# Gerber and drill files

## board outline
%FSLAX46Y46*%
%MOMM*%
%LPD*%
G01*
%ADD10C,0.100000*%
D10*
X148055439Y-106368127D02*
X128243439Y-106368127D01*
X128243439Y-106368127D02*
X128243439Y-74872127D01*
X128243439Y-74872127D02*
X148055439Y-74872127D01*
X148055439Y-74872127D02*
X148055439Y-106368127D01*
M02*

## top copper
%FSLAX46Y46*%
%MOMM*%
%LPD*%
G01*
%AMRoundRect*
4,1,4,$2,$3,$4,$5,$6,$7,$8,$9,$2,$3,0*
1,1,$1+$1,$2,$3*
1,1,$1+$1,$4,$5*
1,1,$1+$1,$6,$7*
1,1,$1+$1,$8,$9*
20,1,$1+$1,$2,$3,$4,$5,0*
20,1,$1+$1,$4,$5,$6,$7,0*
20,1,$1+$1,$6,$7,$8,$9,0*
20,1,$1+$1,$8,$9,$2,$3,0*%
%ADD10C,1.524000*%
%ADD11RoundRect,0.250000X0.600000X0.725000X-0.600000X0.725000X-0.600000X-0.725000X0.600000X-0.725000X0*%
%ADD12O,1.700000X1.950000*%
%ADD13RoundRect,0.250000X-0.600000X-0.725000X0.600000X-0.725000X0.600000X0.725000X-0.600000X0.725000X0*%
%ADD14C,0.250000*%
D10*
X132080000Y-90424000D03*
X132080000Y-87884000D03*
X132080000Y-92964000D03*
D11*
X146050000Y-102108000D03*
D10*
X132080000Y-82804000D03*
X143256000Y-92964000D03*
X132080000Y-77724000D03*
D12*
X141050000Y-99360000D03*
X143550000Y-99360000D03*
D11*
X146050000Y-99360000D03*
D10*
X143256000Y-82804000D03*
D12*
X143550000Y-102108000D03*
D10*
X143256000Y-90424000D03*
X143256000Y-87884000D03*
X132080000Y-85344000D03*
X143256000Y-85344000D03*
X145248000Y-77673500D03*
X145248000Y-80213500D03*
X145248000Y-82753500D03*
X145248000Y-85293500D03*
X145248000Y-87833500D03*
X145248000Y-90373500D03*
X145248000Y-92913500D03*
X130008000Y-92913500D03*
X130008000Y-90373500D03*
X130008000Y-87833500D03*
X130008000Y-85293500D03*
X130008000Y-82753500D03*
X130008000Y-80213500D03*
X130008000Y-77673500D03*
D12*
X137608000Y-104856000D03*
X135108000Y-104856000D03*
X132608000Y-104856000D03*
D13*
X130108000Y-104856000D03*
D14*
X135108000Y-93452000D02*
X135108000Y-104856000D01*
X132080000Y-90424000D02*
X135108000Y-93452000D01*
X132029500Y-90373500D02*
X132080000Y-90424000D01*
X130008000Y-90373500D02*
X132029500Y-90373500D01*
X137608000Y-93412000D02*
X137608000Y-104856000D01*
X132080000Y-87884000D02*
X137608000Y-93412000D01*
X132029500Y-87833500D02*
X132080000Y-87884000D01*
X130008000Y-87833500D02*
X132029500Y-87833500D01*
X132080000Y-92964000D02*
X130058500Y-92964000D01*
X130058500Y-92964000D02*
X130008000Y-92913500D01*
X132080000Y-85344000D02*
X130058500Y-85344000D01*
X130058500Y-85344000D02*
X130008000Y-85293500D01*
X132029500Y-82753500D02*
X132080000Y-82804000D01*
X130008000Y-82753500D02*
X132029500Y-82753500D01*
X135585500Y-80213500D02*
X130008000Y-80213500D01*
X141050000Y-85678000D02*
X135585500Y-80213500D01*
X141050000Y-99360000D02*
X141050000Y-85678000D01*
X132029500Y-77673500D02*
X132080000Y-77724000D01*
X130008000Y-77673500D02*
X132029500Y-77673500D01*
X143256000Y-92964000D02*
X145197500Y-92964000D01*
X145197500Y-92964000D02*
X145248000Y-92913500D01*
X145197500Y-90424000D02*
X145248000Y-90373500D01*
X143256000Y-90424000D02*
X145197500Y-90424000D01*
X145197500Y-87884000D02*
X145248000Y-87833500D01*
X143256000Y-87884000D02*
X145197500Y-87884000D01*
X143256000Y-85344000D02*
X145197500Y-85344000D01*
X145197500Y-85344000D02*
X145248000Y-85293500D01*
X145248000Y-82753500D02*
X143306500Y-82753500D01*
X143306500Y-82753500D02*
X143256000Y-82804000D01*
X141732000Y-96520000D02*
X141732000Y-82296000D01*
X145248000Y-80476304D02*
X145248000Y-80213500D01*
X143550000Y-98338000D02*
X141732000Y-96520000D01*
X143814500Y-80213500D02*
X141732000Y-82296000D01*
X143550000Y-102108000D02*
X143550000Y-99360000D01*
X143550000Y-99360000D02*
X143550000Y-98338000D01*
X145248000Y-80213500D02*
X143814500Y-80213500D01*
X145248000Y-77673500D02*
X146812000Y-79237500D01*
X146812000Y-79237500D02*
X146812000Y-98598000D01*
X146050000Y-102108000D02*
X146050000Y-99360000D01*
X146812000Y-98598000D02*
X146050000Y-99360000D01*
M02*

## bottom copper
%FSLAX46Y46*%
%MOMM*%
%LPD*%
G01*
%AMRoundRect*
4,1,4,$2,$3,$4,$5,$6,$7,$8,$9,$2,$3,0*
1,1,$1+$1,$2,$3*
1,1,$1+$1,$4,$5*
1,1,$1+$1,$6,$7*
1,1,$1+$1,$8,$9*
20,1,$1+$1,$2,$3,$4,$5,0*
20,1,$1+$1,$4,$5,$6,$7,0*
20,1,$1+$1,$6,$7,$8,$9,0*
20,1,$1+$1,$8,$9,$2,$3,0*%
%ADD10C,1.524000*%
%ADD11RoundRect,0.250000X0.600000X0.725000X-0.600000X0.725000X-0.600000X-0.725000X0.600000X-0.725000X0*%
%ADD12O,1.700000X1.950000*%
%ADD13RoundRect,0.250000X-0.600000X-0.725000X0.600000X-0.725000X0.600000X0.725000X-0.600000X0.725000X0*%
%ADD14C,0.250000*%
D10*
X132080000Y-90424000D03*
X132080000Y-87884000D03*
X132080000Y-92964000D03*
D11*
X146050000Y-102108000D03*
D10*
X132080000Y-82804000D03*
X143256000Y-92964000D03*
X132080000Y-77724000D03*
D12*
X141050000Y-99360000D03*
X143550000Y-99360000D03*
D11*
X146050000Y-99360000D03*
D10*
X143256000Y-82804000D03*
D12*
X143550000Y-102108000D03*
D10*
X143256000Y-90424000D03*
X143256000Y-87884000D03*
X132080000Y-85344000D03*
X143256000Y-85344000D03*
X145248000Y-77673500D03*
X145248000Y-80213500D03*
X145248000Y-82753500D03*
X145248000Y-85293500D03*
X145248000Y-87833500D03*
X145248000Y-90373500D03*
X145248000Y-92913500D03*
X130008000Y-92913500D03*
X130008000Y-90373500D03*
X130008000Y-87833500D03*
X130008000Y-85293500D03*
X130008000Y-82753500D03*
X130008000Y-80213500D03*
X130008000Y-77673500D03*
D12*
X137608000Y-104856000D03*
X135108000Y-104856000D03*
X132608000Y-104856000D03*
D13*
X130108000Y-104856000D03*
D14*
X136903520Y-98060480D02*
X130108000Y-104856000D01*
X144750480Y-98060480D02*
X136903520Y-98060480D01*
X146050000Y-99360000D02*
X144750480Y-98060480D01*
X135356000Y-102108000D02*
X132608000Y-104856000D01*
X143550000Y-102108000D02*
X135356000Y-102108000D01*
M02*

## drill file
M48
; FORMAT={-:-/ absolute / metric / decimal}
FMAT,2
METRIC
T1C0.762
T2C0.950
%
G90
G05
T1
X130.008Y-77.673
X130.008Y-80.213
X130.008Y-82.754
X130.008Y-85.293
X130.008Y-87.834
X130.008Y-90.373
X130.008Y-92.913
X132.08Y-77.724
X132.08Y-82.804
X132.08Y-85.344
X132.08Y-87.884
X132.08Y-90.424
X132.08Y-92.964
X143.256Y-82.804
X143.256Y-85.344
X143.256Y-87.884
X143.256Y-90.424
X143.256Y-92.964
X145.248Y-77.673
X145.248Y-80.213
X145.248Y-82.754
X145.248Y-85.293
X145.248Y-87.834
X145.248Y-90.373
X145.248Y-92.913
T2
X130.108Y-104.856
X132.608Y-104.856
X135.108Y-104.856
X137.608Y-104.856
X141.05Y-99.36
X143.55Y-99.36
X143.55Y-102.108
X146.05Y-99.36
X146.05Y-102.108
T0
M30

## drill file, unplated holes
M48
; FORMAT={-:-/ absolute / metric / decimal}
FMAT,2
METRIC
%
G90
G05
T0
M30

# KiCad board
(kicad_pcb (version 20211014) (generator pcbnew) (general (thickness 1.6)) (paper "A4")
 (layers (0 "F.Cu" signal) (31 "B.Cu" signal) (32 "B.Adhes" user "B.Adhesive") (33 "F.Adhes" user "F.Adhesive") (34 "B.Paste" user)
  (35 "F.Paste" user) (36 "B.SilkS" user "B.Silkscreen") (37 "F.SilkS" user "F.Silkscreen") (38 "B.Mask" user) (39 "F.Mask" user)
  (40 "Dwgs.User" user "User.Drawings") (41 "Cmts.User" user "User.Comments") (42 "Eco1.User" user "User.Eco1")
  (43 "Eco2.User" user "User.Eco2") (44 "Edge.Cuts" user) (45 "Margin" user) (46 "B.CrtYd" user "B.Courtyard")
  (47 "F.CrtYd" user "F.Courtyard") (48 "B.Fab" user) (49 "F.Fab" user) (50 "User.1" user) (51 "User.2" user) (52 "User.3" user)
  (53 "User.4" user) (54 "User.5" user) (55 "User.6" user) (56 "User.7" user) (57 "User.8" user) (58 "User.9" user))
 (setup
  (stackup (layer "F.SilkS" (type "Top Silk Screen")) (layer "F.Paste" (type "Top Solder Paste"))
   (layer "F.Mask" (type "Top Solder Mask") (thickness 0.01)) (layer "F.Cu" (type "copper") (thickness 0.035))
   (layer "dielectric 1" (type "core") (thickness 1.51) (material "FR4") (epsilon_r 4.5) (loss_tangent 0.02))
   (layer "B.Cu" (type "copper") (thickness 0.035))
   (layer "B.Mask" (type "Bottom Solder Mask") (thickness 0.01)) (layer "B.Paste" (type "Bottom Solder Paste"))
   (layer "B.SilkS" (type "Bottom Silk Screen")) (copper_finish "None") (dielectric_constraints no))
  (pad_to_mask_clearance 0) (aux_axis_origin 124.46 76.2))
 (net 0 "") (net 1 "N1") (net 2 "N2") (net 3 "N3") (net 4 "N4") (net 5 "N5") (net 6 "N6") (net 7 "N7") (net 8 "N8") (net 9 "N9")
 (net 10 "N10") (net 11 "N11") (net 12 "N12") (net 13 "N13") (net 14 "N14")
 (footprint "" (layer "F.Cu") (at 132.08 92.964)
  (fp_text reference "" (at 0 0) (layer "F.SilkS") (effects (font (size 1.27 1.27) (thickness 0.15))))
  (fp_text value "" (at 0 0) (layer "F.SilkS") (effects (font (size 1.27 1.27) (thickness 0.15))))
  (pad "7" thru_hole circle (at 0 0) (size 1.524 1.524) (drill 0.762) (layers *.Cu *.Mask) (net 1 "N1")))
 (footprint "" (layer "F.Cu") (at 146.05 102.108)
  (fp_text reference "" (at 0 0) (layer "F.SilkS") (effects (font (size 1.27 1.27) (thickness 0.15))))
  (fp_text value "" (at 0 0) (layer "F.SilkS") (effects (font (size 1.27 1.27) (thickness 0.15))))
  (pad "1" thru_hole roundrect (at 0 0 180) (size 1.7 1.95) (drill 0.95) (layers *.Cu *.Mask) (roundrect_rratio 0.1470588235) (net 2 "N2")))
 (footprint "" (layer "F.Cu") (at 132.08 82.804)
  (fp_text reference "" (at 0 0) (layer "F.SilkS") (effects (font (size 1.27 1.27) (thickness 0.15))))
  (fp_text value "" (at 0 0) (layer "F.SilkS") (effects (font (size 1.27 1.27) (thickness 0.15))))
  (pad "3" thru_hole circle (at 0 0) (size 1.524 1.524) (drill 0.762) (layers *.Cu *.Mask) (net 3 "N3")))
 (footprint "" (layer "F.Cu") (at 143.256 92.964)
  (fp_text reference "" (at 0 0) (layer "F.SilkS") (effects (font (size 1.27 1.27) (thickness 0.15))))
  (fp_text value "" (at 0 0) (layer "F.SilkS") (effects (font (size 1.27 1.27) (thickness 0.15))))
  (pad "8" thru_hole circle (at 0 0) (size 1.524 1.524) (drill 0.762) (layers *.Cu *.Mask) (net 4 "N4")))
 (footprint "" (layer "F.Cu") (at 132.08 87.884)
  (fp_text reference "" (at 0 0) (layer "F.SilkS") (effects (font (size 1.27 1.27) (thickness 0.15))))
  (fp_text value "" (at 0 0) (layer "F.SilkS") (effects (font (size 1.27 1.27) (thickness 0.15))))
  (pad "5" thru_hole circle (at 0 0) (size 1.524 1.524) (drill 0.762) (layers *.Cu *.Mask) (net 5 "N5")))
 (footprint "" (layer "F.Cu") (at 132.08 77.724)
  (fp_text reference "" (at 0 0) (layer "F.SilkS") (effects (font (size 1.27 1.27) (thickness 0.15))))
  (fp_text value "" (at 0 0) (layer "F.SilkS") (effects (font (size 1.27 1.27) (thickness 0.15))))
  (pad "1" thru_hole circle (at 0 0) (size 1.524 1.524) (drill 0.762) (layers *.Cu *.Mask) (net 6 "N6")))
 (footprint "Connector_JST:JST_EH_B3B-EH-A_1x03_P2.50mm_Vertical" (layer "F.Cu") (at 146.05 99.36 180)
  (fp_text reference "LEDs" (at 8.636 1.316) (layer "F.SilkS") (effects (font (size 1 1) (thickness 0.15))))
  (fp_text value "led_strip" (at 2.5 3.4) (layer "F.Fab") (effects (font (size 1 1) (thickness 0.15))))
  (pad "1" thru_hole roundrect (at 0 0 180) (size 1.7 1.95) (drill 0.95) (layers *.Cu *.Mask) (roundrect_rratio 0.1470588235) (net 2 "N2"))
  (pad "2" thru_hole oval (at 2.5 0 180) (size 1.7 1.95) (drill 0.95) (layers *.Cu *.Mask) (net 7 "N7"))
  (pad "3" thru_hole oval (at 5 0 180) (size 1.7 1.95) (drill 0.95) (layers *.Cu *.Mask) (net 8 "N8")))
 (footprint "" (layer "F.Cu") (at 143.256 82.804)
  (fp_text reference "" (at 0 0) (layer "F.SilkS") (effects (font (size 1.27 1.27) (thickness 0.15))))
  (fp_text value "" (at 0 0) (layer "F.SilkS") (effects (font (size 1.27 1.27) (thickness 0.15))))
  (pad "12" thru_hole circle (at 0 0) (size 1.524 1.524) (drill 0.762) (layers *.Cu *.Mask) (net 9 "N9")))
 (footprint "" (layer "F.Cu") (at 143.55 102.108)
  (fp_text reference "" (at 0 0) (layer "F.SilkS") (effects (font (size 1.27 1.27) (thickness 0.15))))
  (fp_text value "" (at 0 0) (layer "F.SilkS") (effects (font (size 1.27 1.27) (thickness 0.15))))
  (pad "2" thru_hole oval (at 0 0 180) (size 1.7 1.95) (drill 0.95) (layers *.Cu *.Mask) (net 7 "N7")))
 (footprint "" (layer "F.Cu") (at 143.256 90.424)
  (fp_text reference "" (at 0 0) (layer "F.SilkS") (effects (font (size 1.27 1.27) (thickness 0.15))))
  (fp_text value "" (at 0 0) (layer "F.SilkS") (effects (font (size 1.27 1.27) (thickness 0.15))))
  (pad "9" thru_hole circle (at 0 0) (size 1.524 1.524) (drill 0.762) (layers *.Cu *.Mask) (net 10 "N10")))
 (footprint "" (layer "F.Cu") (at 143.256 87.884)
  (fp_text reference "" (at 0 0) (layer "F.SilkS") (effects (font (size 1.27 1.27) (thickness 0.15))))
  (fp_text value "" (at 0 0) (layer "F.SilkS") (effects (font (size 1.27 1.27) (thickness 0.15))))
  (pad "10" thru_hole circle (at 0 0) (size 1.524 1.524) (drill 0.762) (layers *.Cu *.Mask) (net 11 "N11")))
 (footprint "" (layer "F.Cu") (at 132.08 90.424)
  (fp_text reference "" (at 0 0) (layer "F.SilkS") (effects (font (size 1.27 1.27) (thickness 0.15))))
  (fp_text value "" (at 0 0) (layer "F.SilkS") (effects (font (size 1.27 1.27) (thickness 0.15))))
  (pad "6" thru_hole circle (at 0 0) (size 1.524 1.524) (drill 0.762) (layers *.Cu *.Mask) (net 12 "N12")))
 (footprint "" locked (layer "F.Cu") (at 132.08 85.344)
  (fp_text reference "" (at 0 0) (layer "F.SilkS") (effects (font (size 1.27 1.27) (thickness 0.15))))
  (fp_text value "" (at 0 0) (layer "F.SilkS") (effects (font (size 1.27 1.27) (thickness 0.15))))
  (pad "4" thru_hole circle locked (at 0 0) (size 1.524 1.524) (drill 0.762) (layers *.Cu *.Mask) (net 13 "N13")))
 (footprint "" (layer "F.Cu") (at 143.256 85.344)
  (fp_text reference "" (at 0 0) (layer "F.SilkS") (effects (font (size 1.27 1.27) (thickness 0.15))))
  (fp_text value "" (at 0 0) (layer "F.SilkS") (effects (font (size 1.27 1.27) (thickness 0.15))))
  (pad "11" thru_hole circle (at 0 0) (size 1.524 1.524) (drill 0.762) (layers *.Cu *.Mask) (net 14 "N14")))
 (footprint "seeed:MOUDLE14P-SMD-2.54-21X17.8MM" (layer "F.Cu") (at 130.008 95.7935)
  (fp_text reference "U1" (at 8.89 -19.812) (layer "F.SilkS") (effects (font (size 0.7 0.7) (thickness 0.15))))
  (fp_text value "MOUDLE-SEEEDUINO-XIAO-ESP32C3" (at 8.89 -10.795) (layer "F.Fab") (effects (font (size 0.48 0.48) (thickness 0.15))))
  (pad "1" thru_hole circle (at 0 -18.12) (size 1.524 1.524) (drill 0.762) (layers *.Cu *.Mask) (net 6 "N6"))
  (pad "2" thru_hole circle (at 0 -15.58) (size 1.524 1.524) (drill 0.762) (layers *.Cu *.Mask) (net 8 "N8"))
  (pad "3" thru_hole circle (at 0 -13.04) (size 1.524 1.524) (drill 0.762) (layers *.Cu *.Mask) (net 3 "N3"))
  (pad "4" thru_hole circle (at 0 -10.5) (size 1.524 1.524) (drill 0.762) (layers *.Cu *.Mask) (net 13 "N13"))
  (pad "5" thru_hole circle locked (at 0 -7.96) (size 1.524 1.524) (drill 0.762) (layers *.Cu *.Mask) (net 5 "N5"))
  (pad "6" thru_hole circle (at 0 -5.42) (size 1.524 1.524) (drill 0.762) (layers *.Cu *.Mask) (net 12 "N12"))
  (pad "7" thru_hole circle (at 0 -2.88) (size 1.524 1.524) (drill 0.762) (layers *.Cu *.Mask) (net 1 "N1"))
  (pad "8" thru_hole circle (at 15.24 -2.88) (size 1.524 1.524) (drill 0.762) (layers *.Cu *.Mask) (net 4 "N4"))
  (pad "9" thru_hole circle (at 15.24 -5.42) (size 1.524 1.524) (drill 0.762) (layers *.Cu *.Mask) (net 10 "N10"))
  (pad "10" thru_hole circle (at 15.24 -7.96) (size 1.524 1.524) (drill 0.762) (layers *.Cu *.Mask) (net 11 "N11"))
  (pad "11" thru_hole circle (at 15.24 -10.5) (size 1.524 1.524) (drill 0.762) (layers *.Cu *.Mask) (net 14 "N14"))
  (pad "12" thru_hole circle (at 15.24 -13.04) (size 1.524 1.524) (drill 0.762) (layers *.Cu *.Mask) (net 9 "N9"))
  (pad "13" thru_hole circle (at 15.24 -15.58) (size 1.524 1.524) (drill 0.762) (layers *.Cu *.Mask) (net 7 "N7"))
  (pad "14" thru_hole circle (at 15.24 -18.12) (size 1.524 1.524) (drill 0.762) (layers *.Cu *.Mask) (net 2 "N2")))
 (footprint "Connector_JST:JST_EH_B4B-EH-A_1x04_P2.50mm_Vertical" (layer "F.Cu") (at 130.108 104.856)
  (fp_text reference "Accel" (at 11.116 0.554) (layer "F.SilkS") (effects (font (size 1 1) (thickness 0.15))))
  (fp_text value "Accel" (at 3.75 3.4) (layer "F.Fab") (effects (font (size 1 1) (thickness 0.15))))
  (pad "1" thru_hole roundrect (at 0 0) (size 1.7 1.95) (drill 0.95) (layers *.Cu *.Mask) (roundrect_rratio 0.1470588235) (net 2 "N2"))
  (pad "2" thru_hole oval (at 2.5 0) (size 1.7 1.95) (drill 0.95) (layers *.Cu *.Mask) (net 7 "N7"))
  (pad "3" thru_hole oval (at 5 0) (size 1.7 1.95) (drill 0.95) (layers *.Cu *.Mask) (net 12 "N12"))
  (pad "4" thru_hole oval (at 7.5 0) (size 1.7 1.95) (drill 0.95) (layers *.Cu *.Mask) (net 5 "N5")))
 (gr_rect (start 148.055439 106.368127) (end 128.243439 74.872127) (layer "Edge.Cuts") (width 0.1) (fill none))
 (segment (start 132.08 92.964) (end 130.0585 92.964) (width 0.25) (layer "F.Cu") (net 1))
 (segment (start 130.0585 92.964) (end 130.008 92.9135) (width 0.25) (layer "F.Cu") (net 1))
 (segment (start 132.08 90.424) (end 135.108 93.452) (width 0.25) (layer "F.Cu") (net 12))
 (segment (start 135.108 93.452) (end 135.108 104.856) (width 0.25) (layer "F.Cu") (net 12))
 (segment (start 132.0295 90.3735) (end 132.08 90.424) (width 0.25) (layer "F.Cu") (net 12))
 (segment (start 130.008 90.3735) (end 132.0295 90.3735) (width 0.25) (layer "F.Cu") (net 12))
 (segment (start 132.08 87.884) (end 137.608 93.412) (width 0.25) (layer "F.Cu") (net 5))
 (segment (start 132.0295 87.8335) (end 132.08 87.884) (width 0.25) (layer "F.Cu") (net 5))
 (segment (start 130.008 87.8335) (end 132.0295 87.8335) (width 0.25) (layer "F.Cu") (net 5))
 (segment (start 137.608 93.412) (end 137.608 104.856) (width 0.25) (layer "F.Cu") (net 5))
 (segment (start 132.08 85.344) (end 130.0585 85.344) (width 0.25) (layer "F.Cu") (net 13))
 (segment (start 130.0585 85.344) (end 130.008 85.2935) (width 0.25) (layer "F.Cu") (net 13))
 (segment (start 132.0295 82.7535) (end 132.08 82.804) (width 0.25) (layer "F.Cu") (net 3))
 (segment (start 130.008 82.7535) (end 132.0295 82.7535) (width 0.25) (layer "F.Cu") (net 3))
 (segment (start 135.5855 80.2135) (end 130.008 80.2135) (width 0.25) (layer "F.Cu") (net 8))
 (segment (start 141.05 85.678) (end 135.5855 80.2135) (width 0.25) (layer "F.Cu") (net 8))
 (segment (start 141.05 99.36) (end 141.05 85.678) (width 0.25) (layer "F.Cu") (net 8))
 (segment (start 132.0295 77.6735) (end 132.08 77.724) (width 0.25) (layer "F.Cu") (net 6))
 (segment (start 130.008 77.6735) (end 132.0295 77.6735) (width 0.25) (layer "F.Cu") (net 6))
 (segment (start 143.256 92.964) (end 145.1975 92.964) (width 0.25) (layer "F.Cu") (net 4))
 (segment (start 145.1975 92.964) (end 145.248 92.9135) (width 0.25) (layer "F.Cu") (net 4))
 (segment (start 145.1975 90.424) (end 145.248 90.3735) (width 0.25) (layer "F.Cu") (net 10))
 (segment (start 143.256 90.424) (end 145.1975 90.424) (width 0.25) (layer "F.Cu") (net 10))
 (segment (start 145.1975 87.884) (end 145.248 87.8335) (width 0.25) (layer "F.Cu") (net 11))
 (segment (start 143.256 87.884) (end 145.1975 87.884) (width 0.25) (layer "F.Cu") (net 11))
 (segment (start 143.256 85.344) (end 145.1975 85.344) (width 0.25) (layer "F.Cu") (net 14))
 (segment (start 145.1975 85.344) (end 145.248 85.2935) (width 0.25) (layer "F.Cu") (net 14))
 (segment (start 145.248 82.7535) (end 143.3065 82.7535) (width 0.25) (layer "F.Cu") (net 9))
 (segment (start 143.3065 82.7535) (end 143.256 82.804) (width 0.25) (layer "F.Cu") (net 9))
 (segment (start 141.732 96.52) (end 141.732 82.296) (width 0.25) (layer "F.Cu") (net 7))
 (segment (start 145.248 80.476304) (end 145.248 80.2135) (width 0.25) (layer "F.Cu") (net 7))
 (segment (start 143.55 98.338) (end 141.732 96.52) (width 0.25) (layer "F.Cu") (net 7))
 (segment (start 143.8145 80.2135) (end 141.732 82.296) (width 0.25) (layer "F.Cu") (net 7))
 (segment (start 143.55 102.108) (end 143.55 99.36) (width 0.25) (layer "F.Cu") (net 7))
 (segment (start 143.55 99.36) (end 143.55 98.338) (width 0.25) (layer "F.Cu") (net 7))
 (segment (start 145.248 80.2135) (end 143.8145 80.2135) (width 0.25) (layer "F.Cu") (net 7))
 (segment (start 135.356 102.108) (end 132.608 104.856) (width 0.25) (layer "B.Cu") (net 7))
 (segment (start 143.55 102.108) (end 135.356 102.108) (width 0.25) (layer "B.Cu") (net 7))
 (segment (start 145.248 77.6735) (end 146.812 79.2375) (width 0.25) (layer "F.Cu") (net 2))
 (segment (start 146.812 79.2375) (end 146.812 98.598) (width 0.25) (layer "F.Cu") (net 2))
 (segment (start 146.05 102.108) (end 146.05 99.36) (width 0.25) (layer "F.Cu") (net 2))
 (segment (start 146.812 98.598) (end 146.05 99.36) (width 0.25) (layer "F.Cu") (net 2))
 (segment (start 136.90352 98.06048) (end 130.108 104.856) (width 0.25) (layer "B.Cu") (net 2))
 (segment (start 146.05 99.36) (end 144.75048 98.06048) (width 0.25) (layer "B.Cu") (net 2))
 (segment (start 144.75048 98.06048) (end 136.90352 98.06048) (width 0.25) (layer "B.Cu") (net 2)))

